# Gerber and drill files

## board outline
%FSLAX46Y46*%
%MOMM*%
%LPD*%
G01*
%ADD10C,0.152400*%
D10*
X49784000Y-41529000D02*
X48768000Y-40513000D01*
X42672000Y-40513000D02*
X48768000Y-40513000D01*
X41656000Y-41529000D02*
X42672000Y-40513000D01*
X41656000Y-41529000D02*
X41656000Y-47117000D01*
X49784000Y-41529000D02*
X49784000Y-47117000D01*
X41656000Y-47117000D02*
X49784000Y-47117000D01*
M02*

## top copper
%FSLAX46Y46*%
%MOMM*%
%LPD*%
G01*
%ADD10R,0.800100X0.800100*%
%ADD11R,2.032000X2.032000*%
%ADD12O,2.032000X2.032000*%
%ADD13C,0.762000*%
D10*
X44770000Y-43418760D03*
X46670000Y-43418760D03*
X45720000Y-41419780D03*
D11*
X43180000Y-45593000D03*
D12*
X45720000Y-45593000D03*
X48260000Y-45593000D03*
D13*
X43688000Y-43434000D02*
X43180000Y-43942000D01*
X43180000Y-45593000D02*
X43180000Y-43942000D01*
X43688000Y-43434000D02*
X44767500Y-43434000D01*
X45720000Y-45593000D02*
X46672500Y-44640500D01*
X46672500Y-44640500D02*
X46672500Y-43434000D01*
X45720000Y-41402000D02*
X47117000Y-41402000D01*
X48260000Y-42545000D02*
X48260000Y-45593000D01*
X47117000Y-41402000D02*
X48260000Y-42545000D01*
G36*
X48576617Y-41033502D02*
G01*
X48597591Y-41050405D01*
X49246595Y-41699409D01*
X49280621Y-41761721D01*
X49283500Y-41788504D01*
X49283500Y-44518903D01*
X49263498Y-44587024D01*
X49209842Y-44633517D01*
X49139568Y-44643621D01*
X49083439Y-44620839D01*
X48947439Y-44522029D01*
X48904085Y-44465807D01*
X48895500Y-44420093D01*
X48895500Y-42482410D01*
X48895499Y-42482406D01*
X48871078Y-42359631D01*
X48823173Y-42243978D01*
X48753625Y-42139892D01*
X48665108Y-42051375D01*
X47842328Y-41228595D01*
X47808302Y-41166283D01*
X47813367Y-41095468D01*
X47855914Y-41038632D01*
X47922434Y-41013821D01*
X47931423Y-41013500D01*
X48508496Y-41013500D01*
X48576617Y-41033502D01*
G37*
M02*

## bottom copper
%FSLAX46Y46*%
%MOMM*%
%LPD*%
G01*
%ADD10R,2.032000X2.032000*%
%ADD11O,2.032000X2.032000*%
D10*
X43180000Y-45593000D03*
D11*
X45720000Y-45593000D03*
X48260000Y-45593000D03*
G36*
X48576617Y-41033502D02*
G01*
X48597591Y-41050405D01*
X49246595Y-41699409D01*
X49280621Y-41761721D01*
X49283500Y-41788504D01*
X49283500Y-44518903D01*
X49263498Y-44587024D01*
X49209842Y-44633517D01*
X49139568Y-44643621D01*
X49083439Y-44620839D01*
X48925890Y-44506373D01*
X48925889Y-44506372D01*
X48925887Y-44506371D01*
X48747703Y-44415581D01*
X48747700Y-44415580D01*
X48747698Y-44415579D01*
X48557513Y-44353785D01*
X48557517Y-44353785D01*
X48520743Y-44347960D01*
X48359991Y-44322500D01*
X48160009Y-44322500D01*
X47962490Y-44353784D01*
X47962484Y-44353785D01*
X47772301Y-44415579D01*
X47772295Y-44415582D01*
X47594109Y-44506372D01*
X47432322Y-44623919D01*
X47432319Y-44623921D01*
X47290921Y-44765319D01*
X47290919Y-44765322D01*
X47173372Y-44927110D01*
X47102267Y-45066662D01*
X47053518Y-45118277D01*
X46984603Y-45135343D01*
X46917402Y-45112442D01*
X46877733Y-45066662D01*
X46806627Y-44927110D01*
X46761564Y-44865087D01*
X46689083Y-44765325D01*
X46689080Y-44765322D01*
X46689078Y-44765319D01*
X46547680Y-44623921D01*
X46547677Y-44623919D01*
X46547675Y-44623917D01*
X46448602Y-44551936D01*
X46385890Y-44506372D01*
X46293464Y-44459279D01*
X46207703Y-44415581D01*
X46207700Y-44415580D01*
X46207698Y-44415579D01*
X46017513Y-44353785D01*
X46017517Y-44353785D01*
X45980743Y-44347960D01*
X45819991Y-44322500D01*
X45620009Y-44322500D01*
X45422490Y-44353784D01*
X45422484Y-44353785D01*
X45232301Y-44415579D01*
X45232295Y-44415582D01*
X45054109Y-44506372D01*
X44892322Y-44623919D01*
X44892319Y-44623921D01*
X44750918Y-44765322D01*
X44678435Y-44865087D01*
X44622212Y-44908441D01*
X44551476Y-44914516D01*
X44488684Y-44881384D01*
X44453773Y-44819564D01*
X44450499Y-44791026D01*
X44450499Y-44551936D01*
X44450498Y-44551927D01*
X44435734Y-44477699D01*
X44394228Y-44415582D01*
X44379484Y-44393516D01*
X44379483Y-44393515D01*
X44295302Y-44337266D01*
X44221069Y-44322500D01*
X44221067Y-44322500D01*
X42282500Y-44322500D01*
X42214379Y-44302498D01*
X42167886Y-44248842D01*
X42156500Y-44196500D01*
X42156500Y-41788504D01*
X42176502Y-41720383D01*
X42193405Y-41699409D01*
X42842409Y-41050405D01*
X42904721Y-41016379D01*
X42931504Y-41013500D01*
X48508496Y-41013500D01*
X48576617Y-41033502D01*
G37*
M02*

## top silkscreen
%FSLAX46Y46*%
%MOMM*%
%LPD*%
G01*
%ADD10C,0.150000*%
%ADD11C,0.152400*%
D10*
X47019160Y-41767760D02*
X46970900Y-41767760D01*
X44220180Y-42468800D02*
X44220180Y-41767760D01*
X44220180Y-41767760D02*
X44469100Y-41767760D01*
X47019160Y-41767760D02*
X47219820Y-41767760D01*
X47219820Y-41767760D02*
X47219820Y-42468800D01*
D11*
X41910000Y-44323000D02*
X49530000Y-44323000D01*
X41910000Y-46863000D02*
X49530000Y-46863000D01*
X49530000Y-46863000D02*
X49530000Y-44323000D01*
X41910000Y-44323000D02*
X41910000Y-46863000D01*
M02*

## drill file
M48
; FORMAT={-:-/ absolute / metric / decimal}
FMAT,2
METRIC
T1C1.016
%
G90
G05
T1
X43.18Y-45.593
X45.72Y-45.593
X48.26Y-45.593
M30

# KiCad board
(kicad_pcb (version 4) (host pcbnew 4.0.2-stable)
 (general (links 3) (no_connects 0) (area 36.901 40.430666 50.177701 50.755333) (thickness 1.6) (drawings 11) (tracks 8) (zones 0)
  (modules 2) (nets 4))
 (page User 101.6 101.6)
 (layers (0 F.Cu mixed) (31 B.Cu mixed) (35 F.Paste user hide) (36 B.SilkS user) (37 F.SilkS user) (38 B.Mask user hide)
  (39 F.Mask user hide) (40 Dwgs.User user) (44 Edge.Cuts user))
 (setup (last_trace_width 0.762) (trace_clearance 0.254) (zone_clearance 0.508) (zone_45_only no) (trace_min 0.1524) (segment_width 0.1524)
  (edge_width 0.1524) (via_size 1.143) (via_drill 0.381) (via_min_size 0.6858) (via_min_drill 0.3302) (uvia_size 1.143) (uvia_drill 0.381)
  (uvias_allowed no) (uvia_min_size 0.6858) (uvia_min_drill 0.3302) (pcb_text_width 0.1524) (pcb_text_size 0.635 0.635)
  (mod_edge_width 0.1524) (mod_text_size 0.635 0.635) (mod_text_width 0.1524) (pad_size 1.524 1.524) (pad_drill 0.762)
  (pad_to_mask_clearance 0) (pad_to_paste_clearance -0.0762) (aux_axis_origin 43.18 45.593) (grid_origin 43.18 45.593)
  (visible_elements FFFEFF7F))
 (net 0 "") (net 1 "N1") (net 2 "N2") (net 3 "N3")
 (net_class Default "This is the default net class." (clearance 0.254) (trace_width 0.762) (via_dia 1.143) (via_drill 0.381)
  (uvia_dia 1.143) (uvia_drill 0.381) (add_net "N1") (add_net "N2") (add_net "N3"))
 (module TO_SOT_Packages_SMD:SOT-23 (layer F.Cu) (at 45.72 42.418)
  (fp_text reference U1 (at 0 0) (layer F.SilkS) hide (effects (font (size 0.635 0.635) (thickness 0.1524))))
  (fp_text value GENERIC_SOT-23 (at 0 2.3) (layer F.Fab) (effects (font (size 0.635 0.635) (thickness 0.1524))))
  (fp_line (start 1.29916 -0.65024) (end 1.2509 -0.65024) (layer F.SilkS) (width 0.15))
  (fp_line (start -1.49982 0.0508) (end -1.49982 -0.65024) (layer F.SilkS) (width 0.15))
  (fp_line (start -1.49982 -0.65024) (end -1.2509 -0.65024) (layer F.SilkS) (width 0.15))
  (fp_line (start 1.29916 -0.65024) (end 1.49982 -0.65024) (layer F.SilkS) (width 0.15))
  (fp_line (start 1.49982 -0.65024) (end 1.49982 0.0508) (layer F.SilkS) (width 0.15))
  (pad 1 smd rect (at -0.95 1.00076) (size 0.8001 0.8001) (layers F.Cu F.Paste F.Mask) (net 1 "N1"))
  (pad 2 smd rect (at 0.95 1.00076) (size 0.8001 0.8001) (layers F.Cu F.Paste F.Mask) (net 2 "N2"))
  (pad 3 smd rect (at 0 -0.99822) (size 0.8001 0.8001) (layers F.Cu F.Paste F.Mask) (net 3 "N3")))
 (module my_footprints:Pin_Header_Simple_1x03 (layer F.Cu) (at 43.18 45.593 90)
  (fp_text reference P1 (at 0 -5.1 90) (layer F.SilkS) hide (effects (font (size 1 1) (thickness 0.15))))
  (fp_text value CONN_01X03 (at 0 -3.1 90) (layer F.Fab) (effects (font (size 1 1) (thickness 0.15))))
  (fp_line (start 1.27 -1.27) (end 1.27 6.35) (layer F.SilkS) (width 0.1524))
  (fp_line (start -1.27 -1.27) (end -1.27 6.35) (layer F.SilkS) (width 0.1524))
  (fp_line (start -1.27 6.35) (end 1.27 6.35) (layer F.SilkS) (width 0.1524))
  (fp_line (start 1.27 -1.27) (end -1.27 -1.27) (layer F.SilkS) (width 0.1524))
  (pad 1 thru_hole rect (at 0 0 90) (size 2.032 2.032) (drill 1.016) (layers *.Cu *.Mask) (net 1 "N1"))
  (pad 2 thru_hole oval (at 0 2.54 90) (size 2.032 2.032) (drill 1.016) (layers *.Cu *.Mask) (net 2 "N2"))
  (pad 3 thru_hole oval (at 0 5.08 90) (size 2.032 2.032) (drill 1.016) (layers *.Cu *.Mask) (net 3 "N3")))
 (gr_line (start 49.784 41.529) (end 48.768 40.513) (angle 90) (layer Edge.Cuts) (width 0.1524))
 (gr_line (start 42.672 40.513) (end 48.768 40.513) (angle 90) (layer Edge.Cuts) (width 0.1524))
 (gr_line (start 41.656 41.529) (end 42.672 40.513) (angle 90) (layer Edge.Cuts) (width 0.1524))
 (gr_line (start 41.656 41.529) (end 41.656 47.117) (angle 90) (layer Edge.Cuts) (width 0.1524))
 (gr_line (start 49.784 41.529) (end 49.784 47.117) (angle 90) (layer Edge.Cuts) (width 0.1524))
 (gr_line (start 41.656 47.117) (end 49.784 47.117) (angle 90) (layer Edge.Cuts) (width 0.1524))
 (segment (start 43.688 43.434) (end 43.18 43.942) (width 0.762) (layer F.Cu) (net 1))
 (segment (start 43.18 45.593) (end 43.18 43.942) (width 0.762) (layer F.Cu) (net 1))
 (segment (start 43.688 43.434) (end 44.7675 43.434) (width 0.762) (layer F.Cu) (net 1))
 (segment (start 45.72 45.593) (end 46.6725 44.6405) (width 0.762) (layer F.Cu) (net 2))
 (segment (start 46.6725 44.6405) (end 46.6725 43.434) (width 0.762) (layer F.Cu) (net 2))
 (segment (start 45.72 41.402) (end 47.117 41.402) (width 0.762) (layer F.Cu) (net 3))
 (segment (start 48.26 42.545) (end 48.26 45.593) (width 0.762) (layer F.Cu) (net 3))
 (segment (start 47.117 41.402) (end 48.26 42.545) (width 0.762) (layer F.Cu) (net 3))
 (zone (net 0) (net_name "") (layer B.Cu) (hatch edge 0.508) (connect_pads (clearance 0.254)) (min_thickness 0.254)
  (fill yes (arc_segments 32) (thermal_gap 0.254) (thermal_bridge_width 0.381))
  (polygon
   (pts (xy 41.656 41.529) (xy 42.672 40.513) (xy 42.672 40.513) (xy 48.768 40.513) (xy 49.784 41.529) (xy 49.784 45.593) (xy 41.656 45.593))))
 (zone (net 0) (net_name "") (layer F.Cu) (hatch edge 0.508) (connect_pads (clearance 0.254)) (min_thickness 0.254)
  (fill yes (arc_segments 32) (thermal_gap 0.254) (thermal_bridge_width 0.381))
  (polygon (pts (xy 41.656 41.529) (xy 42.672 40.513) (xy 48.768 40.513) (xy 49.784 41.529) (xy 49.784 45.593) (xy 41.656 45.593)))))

